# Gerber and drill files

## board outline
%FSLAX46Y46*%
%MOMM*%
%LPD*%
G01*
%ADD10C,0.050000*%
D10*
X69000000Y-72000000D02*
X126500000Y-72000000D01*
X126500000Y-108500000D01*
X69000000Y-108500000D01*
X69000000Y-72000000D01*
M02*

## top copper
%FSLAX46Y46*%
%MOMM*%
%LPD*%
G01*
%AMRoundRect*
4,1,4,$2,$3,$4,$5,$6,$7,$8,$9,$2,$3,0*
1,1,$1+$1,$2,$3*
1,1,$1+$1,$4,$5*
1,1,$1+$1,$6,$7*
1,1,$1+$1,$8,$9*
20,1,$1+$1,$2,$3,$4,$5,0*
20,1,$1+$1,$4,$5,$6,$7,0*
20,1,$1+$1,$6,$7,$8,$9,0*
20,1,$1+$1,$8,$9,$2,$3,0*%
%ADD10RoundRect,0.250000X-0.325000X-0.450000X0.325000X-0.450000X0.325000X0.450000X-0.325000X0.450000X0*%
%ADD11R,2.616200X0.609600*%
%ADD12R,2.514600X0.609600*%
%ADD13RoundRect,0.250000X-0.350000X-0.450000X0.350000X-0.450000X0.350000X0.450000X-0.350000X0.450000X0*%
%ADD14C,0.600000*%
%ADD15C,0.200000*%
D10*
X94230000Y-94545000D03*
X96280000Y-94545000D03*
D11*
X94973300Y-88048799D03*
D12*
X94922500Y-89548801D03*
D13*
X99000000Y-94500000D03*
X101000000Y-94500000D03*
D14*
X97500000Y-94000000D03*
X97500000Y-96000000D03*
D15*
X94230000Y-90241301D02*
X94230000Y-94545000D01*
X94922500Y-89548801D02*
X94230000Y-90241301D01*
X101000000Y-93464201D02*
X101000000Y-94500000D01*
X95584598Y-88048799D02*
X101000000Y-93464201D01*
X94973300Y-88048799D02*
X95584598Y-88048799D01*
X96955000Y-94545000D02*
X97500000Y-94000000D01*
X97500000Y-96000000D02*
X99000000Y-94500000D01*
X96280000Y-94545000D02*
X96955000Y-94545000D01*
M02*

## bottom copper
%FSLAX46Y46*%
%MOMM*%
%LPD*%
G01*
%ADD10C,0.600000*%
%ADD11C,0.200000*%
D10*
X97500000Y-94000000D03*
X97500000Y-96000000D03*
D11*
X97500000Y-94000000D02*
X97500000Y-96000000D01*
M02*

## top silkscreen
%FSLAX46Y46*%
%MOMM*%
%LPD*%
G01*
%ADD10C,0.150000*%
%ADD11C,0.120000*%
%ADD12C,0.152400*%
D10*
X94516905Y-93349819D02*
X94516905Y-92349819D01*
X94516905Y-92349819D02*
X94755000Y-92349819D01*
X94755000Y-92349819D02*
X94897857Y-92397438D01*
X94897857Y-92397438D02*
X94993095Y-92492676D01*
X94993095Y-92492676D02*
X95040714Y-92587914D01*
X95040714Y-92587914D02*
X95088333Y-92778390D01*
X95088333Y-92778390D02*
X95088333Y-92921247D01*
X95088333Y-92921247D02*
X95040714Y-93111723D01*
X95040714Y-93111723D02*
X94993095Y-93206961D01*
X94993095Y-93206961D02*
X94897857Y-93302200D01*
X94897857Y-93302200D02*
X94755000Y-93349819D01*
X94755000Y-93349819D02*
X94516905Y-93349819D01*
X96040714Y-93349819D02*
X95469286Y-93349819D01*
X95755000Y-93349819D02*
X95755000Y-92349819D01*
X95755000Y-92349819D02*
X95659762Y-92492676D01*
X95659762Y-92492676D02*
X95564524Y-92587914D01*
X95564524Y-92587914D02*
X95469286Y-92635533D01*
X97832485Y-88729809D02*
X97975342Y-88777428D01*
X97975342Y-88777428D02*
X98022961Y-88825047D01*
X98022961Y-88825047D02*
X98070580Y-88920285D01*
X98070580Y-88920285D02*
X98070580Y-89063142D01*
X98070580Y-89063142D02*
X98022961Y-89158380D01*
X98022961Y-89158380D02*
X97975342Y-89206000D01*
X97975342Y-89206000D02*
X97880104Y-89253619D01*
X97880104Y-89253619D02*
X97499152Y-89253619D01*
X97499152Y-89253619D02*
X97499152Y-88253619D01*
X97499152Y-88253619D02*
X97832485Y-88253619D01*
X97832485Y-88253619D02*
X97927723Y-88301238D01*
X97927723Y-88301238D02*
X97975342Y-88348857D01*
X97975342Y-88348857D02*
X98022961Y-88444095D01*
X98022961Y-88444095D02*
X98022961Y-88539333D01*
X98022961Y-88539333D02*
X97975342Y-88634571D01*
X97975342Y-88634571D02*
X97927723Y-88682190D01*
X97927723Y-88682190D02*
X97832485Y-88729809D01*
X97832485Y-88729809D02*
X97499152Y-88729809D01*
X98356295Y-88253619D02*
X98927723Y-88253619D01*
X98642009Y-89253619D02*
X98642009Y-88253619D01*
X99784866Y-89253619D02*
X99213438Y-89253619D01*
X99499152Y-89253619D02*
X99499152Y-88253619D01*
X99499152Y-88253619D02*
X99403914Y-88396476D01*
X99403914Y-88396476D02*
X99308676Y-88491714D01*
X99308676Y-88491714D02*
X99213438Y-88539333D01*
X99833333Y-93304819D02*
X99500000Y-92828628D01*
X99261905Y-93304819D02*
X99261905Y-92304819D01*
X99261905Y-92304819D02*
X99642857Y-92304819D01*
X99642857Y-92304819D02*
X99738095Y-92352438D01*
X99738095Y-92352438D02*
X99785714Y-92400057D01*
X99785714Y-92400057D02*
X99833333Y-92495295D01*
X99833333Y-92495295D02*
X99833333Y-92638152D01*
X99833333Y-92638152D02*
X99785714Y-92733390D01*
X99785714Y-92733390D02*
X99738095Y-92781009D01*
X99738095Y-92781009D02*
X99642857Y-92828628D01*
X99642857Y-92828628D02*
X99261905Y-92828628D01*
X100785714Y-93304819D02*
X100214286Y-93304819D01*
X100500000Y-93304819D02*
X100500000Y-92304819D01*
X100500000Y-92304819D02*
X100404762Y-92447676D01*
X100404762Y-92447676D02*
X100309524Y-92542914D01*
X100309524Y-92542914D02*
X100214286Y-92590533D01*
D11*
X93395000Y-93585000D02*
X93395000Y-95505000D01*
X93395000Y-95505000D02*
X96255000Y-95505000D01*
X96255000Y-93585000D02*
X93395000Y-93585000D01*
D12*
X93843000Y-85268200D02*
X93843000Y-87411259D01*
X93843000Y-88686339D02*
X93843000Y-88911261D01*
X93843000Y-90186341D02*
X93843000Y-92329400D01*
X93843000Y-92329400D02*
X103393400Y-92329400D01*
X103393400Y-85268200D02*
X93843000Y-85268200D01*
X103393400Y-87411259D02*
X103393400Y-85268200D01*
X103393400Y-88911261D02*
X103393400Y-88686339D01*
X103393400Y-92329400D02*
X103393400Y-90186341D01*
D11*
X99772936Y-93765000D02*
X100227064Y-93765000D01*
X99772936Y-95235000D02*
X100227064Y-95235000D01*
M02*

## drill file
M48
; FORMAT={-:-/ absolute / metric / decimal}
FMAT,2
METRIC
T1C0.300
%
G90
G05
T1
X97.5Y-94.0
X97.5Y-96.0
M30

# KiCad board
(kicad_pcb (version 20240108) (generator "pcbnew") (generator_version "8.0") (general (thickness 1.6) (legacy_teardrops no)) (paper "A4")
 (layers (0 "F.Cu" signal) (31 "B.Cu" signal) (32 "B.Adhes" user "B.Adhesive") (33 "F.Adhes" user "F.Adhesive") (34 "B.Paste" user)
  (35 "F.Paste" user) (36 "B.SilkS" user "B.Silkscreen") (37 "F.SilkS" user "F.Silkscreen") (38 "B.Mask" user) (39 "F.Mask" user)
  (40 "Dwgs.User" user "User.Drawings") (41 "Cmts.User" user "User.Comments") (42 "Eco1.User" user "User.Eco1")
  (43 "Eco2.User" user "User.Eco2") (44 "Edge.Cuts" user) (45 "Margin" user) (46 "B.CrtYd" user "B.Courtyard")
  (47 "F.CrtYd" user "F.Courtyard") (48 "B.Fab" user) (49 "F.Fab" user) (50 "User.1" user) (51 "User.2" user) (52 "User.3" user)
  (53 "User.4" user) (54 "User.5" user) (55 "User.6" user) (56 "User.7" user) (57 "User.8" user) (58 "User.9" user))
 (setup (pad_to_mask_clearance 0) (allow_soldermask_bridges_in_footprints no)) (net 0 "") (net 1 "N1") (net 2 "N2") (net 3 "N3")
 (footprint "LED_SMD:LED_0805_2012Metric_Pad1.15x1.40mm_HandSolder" (layer "F.Cu") (at 95.255 94.545)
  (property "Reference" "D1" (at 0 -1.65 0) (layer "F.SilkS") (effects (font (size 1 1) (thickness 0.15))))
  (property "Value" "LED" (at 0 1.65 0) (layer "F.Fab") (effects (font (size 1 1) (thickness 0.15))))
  (fp_line (start -1.86 -0.96) (end -1.86 0.96) (stroke (width 0.12) (type solid)) (layer "F.SilkS"))
  (fp_line (start -1.86 0.96) (end 1 0.96) (stroke (width 0.12) (type solid)) (layer "F.SilkS"))
  (fp_line (start 1 -0.96) (end -1.86 -0.96) (stroke (width 0.12) (type solid)) (layer "F.SilkS"))
  (pad "1" smd roundrect (at -1.025 0) (size 1.15 1.4) (layers "F.Cu" "F.Paste" "F.Mask") (roundrect_rratio 0.217391) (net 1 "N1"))
  (pad "2" smd roundrect (at 1.025 0) (size 1.15 1.4) (layers "F.Cu" "F.Paste" "F.Mask") (roundrect_rratio 0.217391) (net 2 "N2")))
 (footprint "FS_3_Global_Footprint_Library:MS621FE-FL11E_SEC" (layer "F.Cu") (at 98.6182 88.7988)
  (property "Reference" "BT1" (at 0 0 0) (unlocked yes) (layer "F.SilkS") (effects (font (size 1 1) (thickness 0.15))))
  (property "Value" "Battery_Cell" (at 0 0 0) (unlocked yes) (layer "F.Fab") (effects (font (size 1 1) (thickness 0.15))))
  (fp_line (start -4.7752 -3.5306) (end -4.7752 -1.387541) (stroke (width 0.1524) (type solid)) (layer "F.SilkS"))
  (fp_line (start -4.7752 -0.112461) (end -4.7752 0.112461) (stroke (width 0.1524) (type solid)) (layer "F.SilkS"))
  (fp_line (start -4.7752 1.387541) (end -4.7752 3.5306) (stroke (width 0.1524) (type solid)) (layer "F.SilkS"))
  (fp_line (start -4.7752 3.5306) (end 4.7752 3.5306) (stroke (width 0.1524) (type solid)) (layer "F.SilkS"))
  (fp_line (start 4.7752 -3.5306) (end -4.7752 -3.5306) (stroke (width 0.1524) (type solid)) (layer "F.SilkS"))
  (fp_line (start 4.7752 -1.387541) (end 4.7752 -3.5306) (stroke (width 0.1524) (type solid)) (layer "F.SilkS"))
  (fp_line (start 4.7752 0.112461) (end 4.7752 -0.112461) (stroke (width 0.1524) (type solid)) (layer "F.SilkS"))
  (fp_line (start 4.7752 3.5306) (end 4.7752 1.387541) (stroke (width 0.1524) (type solid)) (layer "F.SilkS"))
  (pad "1" smd rect (at -3.6449 -0.750001) (size 2.6162 0.6096) (layers "F.Cu" "F.Paste" "F.Mask") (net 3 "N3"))
  (pad "2" smd rect (at -3.6957 0.750001) (size 2.5146 0.6096) (layers "F.Cu" "F.Paste" "F.Mask") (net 1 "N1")))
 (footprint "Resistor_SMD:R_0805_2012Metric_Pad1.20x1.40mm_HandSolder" (layer "F.Cu") (at 100 94.5)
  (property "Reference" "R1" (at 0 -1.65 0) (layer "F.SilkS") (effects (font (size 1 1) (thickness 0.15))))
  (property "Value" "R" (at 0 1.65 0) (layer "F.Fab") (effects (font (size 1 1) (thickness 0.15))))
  (fp_line (start -0.227064 -0.735) (end 0.227064 -0.735) (stroke (width 0.12) (type solid)) (layer "F.SilkS"))
  (fp_line (start -0.227064 0.735) (end 0.227064 0.735) (stroke (width 0.12) (type solid)) (layer "F.SilkS"))
  (pad "1" smd roundrect (at -1 0) (size 1.2 1.4) (layers "F.Cu" "F.Paste" "F.Mask") (roundrect_rratio 0.208333) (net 2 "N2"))
  (pad "2" smd roundrect (at 1 0) (size 1.2 1.4) (layers "F.Cu" "F.Paste" "F.Mask") (roundrect_rratio 0.208333) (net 3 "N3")))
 (gr_rect (start 69 72) (end 126.5 108.5) (stroke (width 0.05) (type default)) (fill none) (layer "Edge.Cuts"))
 (segment (start 94.23 90.241301) (end 94.23 94.545) (width 0.2) (layer "F.Cu") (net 1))
 (segment (start 94.9225 89.548801) (end 94.23 90.241301) (width 0.2) (layer "F.Cu") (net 1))
 (segment (start 101 93.464201) (end 101 94.5) (width 0.2) (layer "F.Cu") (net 3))
 (segment (start 95.584598 88.048799) (end 101 93.464201) (width 0.2) (layer "F.Cu") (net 3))
 (segment (start 94.9733 88.048799) (end 95.584598 88.048799) (width 0.2) (layer "F.Cu") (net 3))
 (segment (start 96.955 94.545) (end 97.5 94) (width 0.2) (layer "F.Cu") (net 2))
 (segment (start 97.5 96) (end 99 94.5) (width 0.2) (layer "F.Cu") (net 2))
 (segment (start 96.28 94.545) (end 96.955 94.545) (width 0.2) (layer "F.Cu") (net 2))
 (via (at 97.5 94) (size 0.6) (drill 0.3) (layers "F.Cu" "B.Cu") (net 2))
 (via (at 97.5 96) (size 0.6) (drill 0.3) (layers "F.Cu" "B.Cu") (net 2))
 (segment (start 97.5 94) (end 97.5 96) (width 0.2) (layer "B.Cu") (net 2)))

